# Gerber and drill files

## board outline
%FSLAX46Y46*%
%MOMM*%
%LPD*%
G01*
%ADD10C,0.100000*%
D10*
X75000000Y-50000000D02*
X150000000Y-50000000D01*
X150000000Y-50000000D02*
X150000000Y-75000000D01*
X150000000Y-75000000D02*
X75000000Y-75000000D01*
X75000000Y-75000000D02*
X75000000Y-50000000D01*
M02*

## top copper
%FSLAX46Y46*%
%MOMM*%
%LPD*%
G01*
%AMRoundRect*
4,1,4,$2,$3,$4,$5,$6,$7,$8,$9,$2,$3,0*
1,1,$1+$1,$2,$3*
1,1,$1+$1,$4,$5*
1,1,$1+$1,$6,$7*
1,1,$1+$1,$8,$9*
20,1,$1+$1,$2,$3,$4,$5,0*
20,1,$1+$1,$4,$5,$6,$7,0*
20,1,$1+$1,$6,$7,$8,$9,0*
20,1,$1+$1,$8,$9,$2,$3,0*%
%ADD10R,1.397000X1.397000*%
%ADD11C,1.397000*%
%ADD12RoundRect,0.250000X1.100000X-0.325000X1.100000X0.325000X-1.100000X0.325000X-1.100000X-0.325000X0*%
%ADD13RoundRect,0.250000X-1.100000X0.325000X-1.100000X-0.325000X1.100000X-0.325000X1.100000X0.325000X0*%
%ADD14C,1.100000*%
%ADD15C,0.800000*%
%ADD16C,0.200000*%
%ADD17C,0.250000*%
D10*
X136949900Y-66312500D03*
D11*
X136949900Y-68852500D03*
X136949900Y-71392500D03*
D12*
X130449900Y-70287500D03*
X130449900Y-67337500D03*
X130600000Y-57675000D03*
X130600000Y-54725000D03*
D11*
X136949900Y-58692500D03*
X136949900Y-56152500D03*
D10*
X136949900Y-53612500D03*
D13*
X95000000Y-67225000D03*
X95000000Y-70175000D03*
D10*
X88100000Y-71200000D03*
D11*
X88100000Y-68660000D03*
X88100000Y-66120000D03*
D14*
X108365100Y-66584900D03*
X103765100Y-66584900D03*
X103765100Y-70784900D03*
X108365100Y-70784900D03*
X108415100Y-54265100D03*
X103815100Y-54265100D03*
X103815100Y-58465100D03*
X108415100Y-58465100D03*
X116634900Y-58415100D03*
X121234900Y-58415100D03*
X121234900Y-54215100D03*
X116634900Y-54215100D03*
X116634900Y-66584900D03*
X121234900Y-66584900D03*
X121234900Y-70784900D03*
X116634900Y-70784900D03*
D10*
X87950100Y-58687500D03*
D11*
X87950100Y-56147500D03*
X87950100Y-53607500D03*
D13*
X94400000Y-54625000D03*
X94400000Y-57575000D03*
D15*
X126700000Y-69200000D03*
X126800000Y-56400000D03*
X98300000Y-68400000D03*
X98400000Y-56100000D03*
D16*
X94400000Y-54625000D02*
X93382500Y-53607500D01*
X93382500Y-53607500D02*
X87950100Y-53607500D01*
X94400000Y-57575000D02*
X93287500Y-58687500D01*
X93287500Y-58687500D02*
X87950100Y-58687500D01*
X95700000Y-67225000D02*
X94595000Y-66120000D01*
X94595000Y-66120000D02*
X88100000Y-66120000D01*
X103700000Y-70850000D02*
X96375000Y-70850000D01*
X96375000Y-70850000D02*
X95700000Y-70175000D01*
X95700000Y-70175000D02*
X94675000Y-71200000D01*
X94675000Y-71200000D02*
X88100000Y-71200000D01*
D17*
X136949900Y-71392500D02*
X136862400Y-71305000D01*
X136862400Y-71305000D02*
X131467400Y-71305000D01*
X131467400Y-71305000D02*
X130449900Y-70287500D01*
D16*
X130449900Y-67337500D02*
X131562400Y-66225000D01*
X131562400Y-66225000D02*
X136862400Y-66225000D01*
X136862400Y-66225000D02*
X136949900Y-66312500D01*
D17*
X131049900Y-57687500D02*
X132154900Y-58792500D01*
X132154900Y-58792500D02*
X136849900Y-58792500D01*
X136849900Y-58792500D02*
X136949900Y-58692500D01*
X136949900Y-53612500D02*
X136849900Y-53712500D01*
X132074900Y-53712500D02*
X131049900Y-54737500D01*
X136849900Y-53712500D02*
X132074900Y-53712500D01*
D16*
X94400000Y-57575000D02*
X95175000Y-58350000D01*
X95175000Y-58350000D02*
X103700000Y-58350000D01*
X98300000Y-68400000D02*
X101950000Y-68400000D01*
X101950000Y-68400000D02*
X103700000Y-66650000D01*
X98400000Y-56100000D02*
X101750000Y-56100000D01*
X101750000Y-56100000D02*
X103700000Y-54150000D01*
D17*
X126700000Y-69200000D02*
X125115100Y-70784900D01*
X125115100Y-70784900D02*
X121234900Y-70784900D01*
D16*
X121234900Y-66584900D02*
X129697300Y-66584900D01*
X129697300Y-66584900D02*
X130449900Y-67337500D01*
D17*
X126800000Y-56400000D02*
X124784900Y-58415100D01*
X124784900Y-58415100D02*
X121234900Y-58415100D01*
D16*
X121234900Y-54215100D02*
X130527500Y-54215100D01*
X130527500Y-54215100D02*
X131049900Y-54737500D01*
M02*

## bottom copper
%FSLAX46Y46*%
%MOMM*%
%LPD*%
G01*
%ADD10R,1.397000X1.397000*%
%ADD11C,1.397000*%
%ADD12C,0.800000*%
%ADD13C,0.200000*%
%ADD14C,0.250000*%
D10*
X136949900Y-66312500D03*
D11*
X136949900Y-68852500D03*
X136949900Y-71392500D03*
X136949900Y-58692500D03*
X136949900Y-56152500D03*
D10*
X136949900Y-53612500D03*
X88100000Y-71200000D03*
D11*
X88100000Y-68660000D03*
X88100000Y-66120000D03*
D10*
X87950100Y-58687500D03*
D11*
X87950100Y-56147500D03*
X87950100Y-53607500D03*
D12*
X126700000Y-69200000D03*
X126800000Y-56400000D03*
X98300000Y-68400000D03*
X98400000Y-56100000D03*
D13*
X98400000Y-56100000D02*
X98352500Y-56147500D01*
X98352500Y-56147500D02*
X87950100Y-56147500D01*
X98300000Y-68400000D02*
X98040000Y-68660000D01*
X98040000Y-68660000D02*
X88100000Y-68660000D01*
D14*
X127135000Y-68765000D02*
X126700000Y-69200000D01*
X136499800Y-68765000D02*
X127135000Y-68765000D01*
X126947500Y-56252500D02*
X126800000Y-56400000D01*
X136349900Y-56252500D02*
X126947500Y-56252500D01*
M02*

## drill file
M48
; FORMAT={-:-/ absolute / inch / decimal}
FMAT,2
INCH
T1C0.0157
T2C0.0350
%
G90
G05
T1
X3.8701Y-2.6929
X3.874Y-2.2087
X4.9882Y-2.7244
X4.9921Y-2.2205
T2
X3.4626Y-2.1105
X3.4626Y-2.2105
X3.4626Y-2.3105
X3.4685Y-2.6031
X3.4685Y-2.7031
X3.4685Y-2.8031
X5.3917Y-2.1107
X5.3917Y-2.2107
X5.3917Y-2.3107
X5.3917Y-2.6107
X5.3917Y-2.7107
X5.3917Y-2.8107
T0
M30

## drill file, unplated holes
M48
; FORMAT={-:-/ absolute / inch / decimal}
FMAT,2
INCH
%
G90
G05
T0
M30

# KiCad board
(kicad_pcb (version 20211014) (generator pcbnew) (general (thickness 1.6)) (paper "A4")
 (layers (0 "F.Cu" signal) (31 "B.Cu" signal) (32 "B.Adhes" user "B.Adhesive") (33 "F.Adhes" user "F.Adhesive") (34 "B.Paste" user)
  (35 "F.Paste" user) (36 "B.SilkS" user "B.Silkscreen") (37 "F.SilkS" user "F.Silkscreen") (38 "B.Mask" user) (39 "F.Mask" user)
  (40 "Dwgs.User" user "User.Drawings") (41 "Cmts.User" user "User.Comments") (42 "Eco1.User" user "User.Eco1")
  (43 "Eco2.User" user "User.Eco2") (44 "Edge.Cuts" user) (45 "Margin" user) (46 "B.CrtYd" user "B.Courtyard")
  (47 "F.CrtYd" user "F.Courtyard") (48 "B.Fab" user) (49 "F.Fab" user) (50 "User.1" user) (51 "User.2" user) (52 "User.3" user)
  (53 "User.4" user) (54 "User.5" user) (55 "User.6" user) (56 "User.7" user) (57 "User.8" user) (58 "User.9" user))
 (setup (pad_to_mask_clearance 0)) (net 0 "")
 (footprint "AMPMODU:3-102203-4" (layer "F.Cu") (at 87.9501 58.6875 90)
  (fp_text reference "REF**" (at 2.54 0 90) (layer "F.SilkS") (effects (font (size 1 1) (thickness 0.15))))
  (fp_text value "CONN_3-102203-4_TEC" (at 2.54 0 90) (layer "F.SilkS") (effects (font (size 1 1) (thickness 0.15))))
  (pad "1" thru_hole rect locked (at 0 0 90) (size 1.397 1.397) (drill 0.889) (layers *.Cu *.Mask))
  (pad "2" thru_hole circle locked (at 2.54 0 90) (size 1.397 1.397) (drill 0.889) (layers *.Cu *.Mask))
  (pad "3" thru_hole circle locked (at 5.08 0 90) (size 1.397 1.397) (drill 0.889) (layers *.Cu *.Mask)))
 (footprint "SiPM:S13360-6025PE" (layer "F.Cu") (at 106.3151 68.6849)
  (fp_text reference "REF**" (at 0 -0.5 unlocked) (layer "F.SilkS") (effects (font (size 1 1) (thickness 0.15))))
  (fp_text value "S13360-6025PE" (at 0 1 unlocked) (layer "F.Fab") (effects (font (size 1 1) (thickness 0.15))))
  (pad "1" smd circle (at 2.05 -2.1) (size 1.1 1.1) (layers "F.Cu" "F.Paste" "F.Mask"))
  (pad "2" smd circle (at -2.55 -2.1) (size 1.1 1.1) (layers "F.Cu" "F.Paste" "F.Mask"))
  (pad "3" smd circle (at -2.55 2.1) (size 1.1 1.1) (layers "F.Cu" "F.Paste" "F.Mask"))
  (pad "4" smd circle (at 2.05 2.1) (size 1.1 1.1) (layers "F.Cu" "F.Paste" "F.Mask")))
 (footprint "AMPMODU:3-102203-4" (layer "F.Cu") (at 136.9499 53.6125 -90)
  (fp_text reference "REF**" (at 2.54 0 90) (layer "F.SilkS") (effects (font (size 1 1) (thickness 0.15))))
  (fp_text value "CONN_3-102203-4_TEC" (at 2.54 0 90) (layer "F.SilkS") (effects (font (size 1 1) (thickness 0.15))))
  (pad "1" thru_hole rect locked (at 0 0 270) (size 1.397 1.397) (drill 0.889) (layers *.Cu *.Mask))
  (pad "2" thru_hole circle locked (at 2.54 0 270) (size 1.397 1.397) (drill 0.889) (layers *.Cu *.Mask))
  (pad "3" thru_hole circle locked (at 5.08 0 270) (size 1.397 1.397) (drill 0.889) (layers *.Cu *.Mask)))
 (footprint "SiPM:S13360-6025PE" (layer "F.Cu") (at 106.3651 56.3651)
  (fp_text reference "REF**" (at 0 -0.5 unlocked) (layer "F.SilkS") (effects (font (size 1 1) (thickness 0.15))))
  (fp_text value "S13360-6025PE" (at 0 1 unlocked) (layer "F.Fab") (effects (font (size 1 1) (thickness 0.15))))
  (pad "1" smd circle (at 2.05 -2.1) (size 1.1 1.1) (layers "F.Cu" "F.Paste" "F.Mask"))
  (pad "2" smd circle (at -2.55 -2.1) (size 1.1 1.1) (layers "F.Cu" "F.Paste" "F.Mask"))
  (pad "3" smd circle (at -2.55 2.1) (size 1.1 1.1) (layers "F.Cu" "F.Paste" "F.Mask"))
  (pad "4" smd circle (at 2.05 2.1) (size 1.1 1.1) (layers "F.Cu" "F.Paste" "F.Mask")))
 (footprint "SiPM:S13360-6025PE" (layer "F.Cu") (at 118.6849 56.3151 180)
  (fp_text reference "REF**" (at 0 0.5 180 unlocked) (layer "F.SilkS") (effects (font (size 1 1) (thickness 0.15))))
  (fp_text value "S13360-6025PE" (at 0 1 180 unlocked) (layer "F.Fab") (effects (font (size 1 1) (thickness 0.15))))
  (pad "1" smd circle (at 2.05 -2.1 180) (size 1.1 1.1) (layers "F.Cu" "F.Paste" "F.Mask"))
  (pad "2" smd circle (at -2.55 -2.1 180) (size 1.1 1.1) (layers "F.Cu" "F.Paste" "F.Mask"))
  (pad "3" smd circle (at -2.55 2.1 180) (size 1.1 1.1) (layers "F.Cu" "F.Paste" "F.Mask"))
  (pad "4" smd circle (at 2.05 2.1 180) (size 1.1 1.1) (layers "F.Cu" "F.Paste" "F.Mask")))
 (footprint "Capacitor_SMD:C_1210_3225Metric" (layer "F.Cu") (at 130.6 56.2 90)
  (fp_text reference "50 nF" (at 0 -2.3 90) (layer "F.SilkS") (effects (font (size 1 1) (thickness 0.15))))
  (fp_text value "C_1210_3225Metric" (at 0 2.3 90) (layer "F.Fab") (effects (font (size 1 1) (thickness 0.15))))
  (pad "1" smd roundrect (at -1.475 0 90) (size 1.15 2.7) (layers "F.Cu" "F.Paste" "F.Mask") (roundrect_rratio 0.2173913043))
  (pad "2" smd roundrect (at 1.475 0 90) (size 1.15 2.7) (layers "F.Cu" "F.Paste" "F.Mask") (roundrect_rratio 0.2173913043)))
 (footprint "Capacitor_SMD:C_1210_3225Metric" (layer "F.Cu") (at 95 68.7 -90)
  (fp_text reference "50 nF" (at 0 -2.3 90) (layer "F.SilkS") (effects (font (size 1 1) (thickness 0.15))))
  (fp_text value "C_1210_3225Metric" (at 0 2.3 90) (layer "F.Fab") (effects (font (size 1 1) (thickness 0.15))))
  (pad "1" smd roundrect (at -1.475 0 270) (size 1.15 2.7) (layers "F.Cu" "F.Paste" "F.Mask") (roundrect_rratio 0.2173913043))
  (pad "2" smd roundrect (at 1.475 0 270) (size 1.15 2.7) (layers "F.Cu" "F.Paste" "F.Mask") (roundrect_rratio 0.2173913043)))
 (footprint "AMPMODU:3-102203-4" (layer "F.Cu") (at 136.9499 66.3125 -90)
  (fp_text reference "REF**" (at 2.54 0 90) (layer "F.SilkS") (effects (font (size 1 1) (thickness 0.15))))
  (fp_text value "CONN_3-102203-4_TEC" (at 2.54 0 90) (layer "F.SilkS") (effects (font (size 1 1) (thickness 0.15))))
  (pad "1" thru_hole rect locked (at 0 0 270) (size 1.397 1.397) (drill 0.889) (layers *.Cu *.Mask))
  (pad "2" thru_hole circle locked (at 2.54 0 270) (size 1.397 1.397) (drill 0.889) (layers *.Cu *.Mask))
  (pad "3" thru_hole circle locked (at 5.08 0 270) (size 1.397 1.397) (drill 0.889) (layers *.Cu *.Mask)))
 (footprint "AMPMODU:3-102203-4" (layer "F.Cu") (at 88.1 71.2 90)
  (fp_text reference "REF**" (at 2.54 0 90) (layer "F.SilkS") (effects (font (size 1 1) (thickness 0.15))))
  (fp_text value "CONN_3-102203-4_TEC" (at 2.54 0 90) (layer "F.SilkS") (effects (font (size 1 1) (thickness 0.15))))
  (pad "1" thru_hole rect locked (at 0 0 90) (size 1.397 1.397) (drill 0.889) (layers *.Cu *.Mask))
  (pad "2" thru_hole circle locked (at 2.54 0 90) (size 1.397 1.397) (drill 0.889) (layers *.Cu *.Mask))
  (pad "3" thru_hole circle locked (at 5.08 0 90) (size 1.397 1.397) (drill 0.889) (layers *.Cu *.Mask)))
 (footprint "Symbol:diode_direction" (layer "F.Cu") (at 123.6 68.9 -90)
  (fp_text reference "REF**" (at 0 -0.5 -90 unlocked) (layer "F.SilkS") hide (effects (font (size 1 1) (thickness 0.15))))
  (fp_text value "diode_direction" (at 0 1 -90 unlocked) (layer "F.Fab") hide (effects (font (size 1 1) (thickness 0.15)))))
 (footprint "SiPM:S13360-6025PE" (layer "F.Cu") (at 118.6849 68.6849 180)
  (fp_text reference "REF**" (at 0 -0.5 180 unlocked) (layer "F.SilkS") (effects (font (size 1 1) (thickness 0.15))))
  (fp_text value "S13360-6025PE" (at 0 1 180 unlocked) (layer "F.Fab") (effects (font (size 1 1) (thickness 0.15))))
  (pad "1" smd circle (at 2.05 -2.1 180) (size 1.1 1.1) (layers "F.Cu" "F.Paste" "F.Mask"))
  (pad "2" smd circle (at -2.55 -2.1 180) (size 1.1 1.1) (layers "F.Cu" "F.Paste" "F.Mask"))
  (pad "3" smd circle (at -2.55 2.1 180) (size 1.1 1.1) (layers "F.Cu" "F.Paste" "F.Mask"))
  (pad "4" smd circle (at 2.05 2.1 180) (size 1.1 1.1) (layers "F.Cu" "F.Paste" "F.Mask")))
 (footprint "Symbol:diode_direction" (layer "F.Cu") (at 123.7 56.5 -90)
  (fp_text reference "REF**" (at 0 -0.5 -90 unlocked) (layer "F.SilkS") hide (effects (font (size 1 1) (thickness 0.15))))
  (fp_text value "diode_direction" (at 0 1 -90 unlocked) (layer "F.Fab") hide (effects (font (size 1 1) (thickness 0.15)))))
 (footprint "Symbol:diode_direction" (layer "F.Cu") (at 101.1 68.8 90)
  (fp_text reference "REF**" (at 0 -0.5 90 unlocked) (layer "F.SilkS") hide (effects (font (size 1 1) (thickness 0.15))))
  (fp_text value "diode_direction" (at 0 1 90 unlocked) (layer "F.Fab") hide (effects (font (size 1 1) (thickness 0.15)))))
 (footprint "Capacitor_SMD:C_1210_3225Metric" (layer "F.Cu") (at 94.4 56.1 -90)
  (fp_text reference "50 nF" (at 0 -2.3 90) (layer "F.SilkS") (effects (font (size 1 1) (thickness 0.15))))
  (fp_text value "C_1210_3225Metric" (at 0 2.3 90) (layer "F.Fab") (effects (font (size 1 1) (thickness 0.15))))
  (pad "1" smd roundrect (at -1.475 0 270) (size 1.15 2.7) (layers "F.Cu" "F.Paste" "F.Mask") (roundrect_rratio 0.2173913043))
  (pad "2" smd roundrect (at 1.475 0 270) (size 1.15 2.7) (layers "F.Cu" "F.Paste" "F.Mask") (roundrect_rratio 0.2173913043)))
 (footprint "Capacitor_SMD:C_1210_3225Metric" (layer "F.Cu") (at 130.4499 68.8125 90)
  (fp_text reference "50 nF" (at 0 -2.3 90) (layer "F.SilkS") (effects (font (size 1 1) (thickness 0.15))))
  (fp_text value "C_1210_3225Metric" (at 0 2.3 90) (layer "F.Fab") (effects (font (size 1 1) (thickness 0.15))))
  (pad "1" smd roundrect (at -1.475 0 90) (size 1.15 2.7) (layers "F.Cu" "F.Paste" "F.Mask") (roundrect_rratio 0.2173913043))
  (pad "2" smd roundrect (at 1.475 0 90) (size 1.15 2.7) (layers "F.Cu" "F.Paste" "F.Mask") (roundrect_rratio 0.2173913043)))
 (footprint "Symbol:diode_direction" (layer "F.Cu") (at 101.4 56.2 90)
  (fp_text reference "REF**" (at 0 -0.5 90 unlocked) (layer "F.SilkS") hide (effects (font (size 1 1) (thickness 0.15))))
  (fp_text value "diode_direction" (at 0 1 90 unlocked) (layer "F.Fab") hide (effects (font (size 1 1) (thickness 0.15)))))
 (gr_rect (start 75 50) (end 150 75) (layer "Edge.Cuts") (width 0.1) (fill none))
 (segment (start 126.7 69.2) (end 125.1151 70.7849) (width 0.25) (layer "F.Cu") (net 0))
 (segment (start 103.7 70.85) (end 96.375 70.85) (width 0.2) (layer "F.Cu") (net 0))
 (segment (start 132.0749 53.7125) (end 131.0499 54.7375) (width 0.25) (layer "F.Cu") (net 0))
 (segment (start 131.0499 57.6875) (end 132.1549 58.7925) (width 0.25) (layer "F.Cu") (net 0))
 (segment (start 131.5624 66.225) (end 136.8624 66.225) (width 0.2) (layer "F.Cu") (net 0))
 (segment (start 136.8499 53.7125) (end 132.0749 53.7125) (width 0.25) (layer "F.Cu") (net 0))
 (segment (start 94.4 57.575) (end 93.2875 58.6875) (width 0.2) (layer "F.Cu") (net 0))
 (segment (start 124.7849 58.4151) (end 121.2349 58.4151) (width 0.25) (layer "F.Cu") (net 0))
 (segment (start 121.2349 54.2151) (end 130.5275 54.2151) (width 0.2) (layer "F.Cu") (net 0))
 (segment (start 129.6973 66.5849) (end 130.4499 67.3375) (width 0.2) (layer "F.Cu") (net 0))
 (segment (start 96.375 70.85) (end 95.7 70.175) (width 0.2) (layer "F.Cu") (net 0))
 (segment (start 101.95 68.4) (end 103.7 66.65) (width 0.2) (layer "F.Cu") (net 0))
 (segment (start 95.7 67.225) (end 94.595 66.12) (width 0.2) (layer "F.Cu") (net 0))
 (segment (start 136.9499 71.3925) (end 136.8624 71.305) (width 0.25) (layer "F.Cu") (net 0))
 (segment (start 101.75 56.1) (end 103.7 54.15) (width 0.2) (layer "F.Cu") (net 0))
 (segment (start 136.8624 66.225) (end 136.9499 66.3125) (width 0.2) (layer "F.Cu") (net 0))
 (segment (start 95.7 70.175) (end 94.675 71.2) (width 0.2) (layer "F.Cu") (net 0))
 (segment (start 94.4 57.575) (end 95.175 58.35) (width 0.2) (layer "F.Cu") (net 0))
 (segment (start 136.8499 58.7925) (end 136.9499 58.6925) (width 0.25) (layer "F.Cu") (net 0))
 (segment (start 136.8624 71.305) (end 131.4674 71.305) (width 0.25) (layer "F.Cu") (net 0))
 (segment (start 136.9499 53.6125) (end 136.8499 53.7125) (width 0.25) (layer "F.Cu") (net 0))
 (segment (start 131.4674 71.305) (end 130.4499 70.2875) (width 0.25) (layer "F.Cu") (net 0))
 (segment (start 125.1151 70.7849) (end 121.2349 70.7849) (width 0.25) (layer "F.Cu") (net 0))
 (segment (start 121.2349 66.5849) (end 129.6973 66.5849) (width 0.2) (layer "F.Cu") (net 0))
 (segment (start 94.675 71.2) (end 88.1 71.2) (width 0.2) (layer "F.Cu") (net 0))
 (segment (start 130.4499 67.3375) (end 131.5624 66.225) (width 0.2) (layer "F.Cu") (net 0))
 (segment (start 130.5275 54.2151) (end 131.0499 54.7375) (width 0.2) (layer "F.Cu") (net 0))
 (segment (start 94.595 66.12) (end 88.1 66.12) (width 0.2) (layer "F.Cu") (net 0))
 (segment (start 93.2875 58.6875) (end 87.9501 58.6875) (width 0.2) (layer "F.Cu") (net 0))
 (segment (start 98.4 56.1) (end 101.75 56.1) (width 0.2) (layer "F.Cu") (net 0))
 (segment (start 93.3825 53.6075) (end 87.9501 53.6075) (width 0.2) (layer "F.Cu") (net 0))
 (segment (start 94.4 54.625) (end 93.3825 53.6075) (width 0.2) (layer "F.Cu") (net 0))
 (segment (start 132.1549 58.7925) (end 136.8499 58.7925) (width 0.25) (layer "F.Cu") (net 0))
 (segment (start 98.3 68.4) (end 101.95 68.4) (width 0.2) (layer "F.Cu") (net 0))
 (segment (start 95.175 58.35) (end 103.7 58.35) (width 0.2) (layer "F.Cu") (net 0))
 (segment (start 126.8 56.4) (end 124.7849 58.4151) (width 0.25) (layer "F.Cu") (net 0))
 (via (at 98.3 68.4) (size 0.8) (drill 0.4) (layers "F.Cu" "B.Cu") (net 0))
 (via (at 98.4 56.1) (size 0.8) (drill 0.4) (layers "F.Cu" "B.Cu") (free) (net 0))
 (via (at 126.7 69.2) (size 0.8) (drill 0.4) (layers "F.Cu" "B.Cu") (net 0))
 (via (at 126.8 56.4) (size 0.8) (drill 0.4) (layers "F.Cu" "B.Cu") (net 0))
 (segment (start 136.4998 68.765) (end 127.135 68.765) (width 0.25) (layer "B.Cu") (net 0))
 (segment (start 98.3525 56.1475) (end 87.9501 56.1475) (width 0.2) (layer "B.Cu") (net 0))
 (segment (start 98.04 68.66) (end 88.1 68.66) (width 0.2) (layer "B.Cu") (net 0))
 (segment (start 126.9475 56.2525) (end 126.8 56.4) (width 0.25) (layer "B.Cu") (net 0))
 (segment (start 98.4 56.1) (end 98.3525 56.1475) (width 0.2) (layer "B.Cu") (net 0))
 (segment (start 98.3 68.4) (end 98.04 68.66) (width 0.2) (layer "B.Cu") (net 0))
 (segment (start 127.135 68.765) (end 126.7 69.2) (width 0.25) (layer "B.Cu") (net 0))
 (segment (start 136.3499 56.2525) (end 126.9475 56.2525) (width 0.25) (layer "B.Cu") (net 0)))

